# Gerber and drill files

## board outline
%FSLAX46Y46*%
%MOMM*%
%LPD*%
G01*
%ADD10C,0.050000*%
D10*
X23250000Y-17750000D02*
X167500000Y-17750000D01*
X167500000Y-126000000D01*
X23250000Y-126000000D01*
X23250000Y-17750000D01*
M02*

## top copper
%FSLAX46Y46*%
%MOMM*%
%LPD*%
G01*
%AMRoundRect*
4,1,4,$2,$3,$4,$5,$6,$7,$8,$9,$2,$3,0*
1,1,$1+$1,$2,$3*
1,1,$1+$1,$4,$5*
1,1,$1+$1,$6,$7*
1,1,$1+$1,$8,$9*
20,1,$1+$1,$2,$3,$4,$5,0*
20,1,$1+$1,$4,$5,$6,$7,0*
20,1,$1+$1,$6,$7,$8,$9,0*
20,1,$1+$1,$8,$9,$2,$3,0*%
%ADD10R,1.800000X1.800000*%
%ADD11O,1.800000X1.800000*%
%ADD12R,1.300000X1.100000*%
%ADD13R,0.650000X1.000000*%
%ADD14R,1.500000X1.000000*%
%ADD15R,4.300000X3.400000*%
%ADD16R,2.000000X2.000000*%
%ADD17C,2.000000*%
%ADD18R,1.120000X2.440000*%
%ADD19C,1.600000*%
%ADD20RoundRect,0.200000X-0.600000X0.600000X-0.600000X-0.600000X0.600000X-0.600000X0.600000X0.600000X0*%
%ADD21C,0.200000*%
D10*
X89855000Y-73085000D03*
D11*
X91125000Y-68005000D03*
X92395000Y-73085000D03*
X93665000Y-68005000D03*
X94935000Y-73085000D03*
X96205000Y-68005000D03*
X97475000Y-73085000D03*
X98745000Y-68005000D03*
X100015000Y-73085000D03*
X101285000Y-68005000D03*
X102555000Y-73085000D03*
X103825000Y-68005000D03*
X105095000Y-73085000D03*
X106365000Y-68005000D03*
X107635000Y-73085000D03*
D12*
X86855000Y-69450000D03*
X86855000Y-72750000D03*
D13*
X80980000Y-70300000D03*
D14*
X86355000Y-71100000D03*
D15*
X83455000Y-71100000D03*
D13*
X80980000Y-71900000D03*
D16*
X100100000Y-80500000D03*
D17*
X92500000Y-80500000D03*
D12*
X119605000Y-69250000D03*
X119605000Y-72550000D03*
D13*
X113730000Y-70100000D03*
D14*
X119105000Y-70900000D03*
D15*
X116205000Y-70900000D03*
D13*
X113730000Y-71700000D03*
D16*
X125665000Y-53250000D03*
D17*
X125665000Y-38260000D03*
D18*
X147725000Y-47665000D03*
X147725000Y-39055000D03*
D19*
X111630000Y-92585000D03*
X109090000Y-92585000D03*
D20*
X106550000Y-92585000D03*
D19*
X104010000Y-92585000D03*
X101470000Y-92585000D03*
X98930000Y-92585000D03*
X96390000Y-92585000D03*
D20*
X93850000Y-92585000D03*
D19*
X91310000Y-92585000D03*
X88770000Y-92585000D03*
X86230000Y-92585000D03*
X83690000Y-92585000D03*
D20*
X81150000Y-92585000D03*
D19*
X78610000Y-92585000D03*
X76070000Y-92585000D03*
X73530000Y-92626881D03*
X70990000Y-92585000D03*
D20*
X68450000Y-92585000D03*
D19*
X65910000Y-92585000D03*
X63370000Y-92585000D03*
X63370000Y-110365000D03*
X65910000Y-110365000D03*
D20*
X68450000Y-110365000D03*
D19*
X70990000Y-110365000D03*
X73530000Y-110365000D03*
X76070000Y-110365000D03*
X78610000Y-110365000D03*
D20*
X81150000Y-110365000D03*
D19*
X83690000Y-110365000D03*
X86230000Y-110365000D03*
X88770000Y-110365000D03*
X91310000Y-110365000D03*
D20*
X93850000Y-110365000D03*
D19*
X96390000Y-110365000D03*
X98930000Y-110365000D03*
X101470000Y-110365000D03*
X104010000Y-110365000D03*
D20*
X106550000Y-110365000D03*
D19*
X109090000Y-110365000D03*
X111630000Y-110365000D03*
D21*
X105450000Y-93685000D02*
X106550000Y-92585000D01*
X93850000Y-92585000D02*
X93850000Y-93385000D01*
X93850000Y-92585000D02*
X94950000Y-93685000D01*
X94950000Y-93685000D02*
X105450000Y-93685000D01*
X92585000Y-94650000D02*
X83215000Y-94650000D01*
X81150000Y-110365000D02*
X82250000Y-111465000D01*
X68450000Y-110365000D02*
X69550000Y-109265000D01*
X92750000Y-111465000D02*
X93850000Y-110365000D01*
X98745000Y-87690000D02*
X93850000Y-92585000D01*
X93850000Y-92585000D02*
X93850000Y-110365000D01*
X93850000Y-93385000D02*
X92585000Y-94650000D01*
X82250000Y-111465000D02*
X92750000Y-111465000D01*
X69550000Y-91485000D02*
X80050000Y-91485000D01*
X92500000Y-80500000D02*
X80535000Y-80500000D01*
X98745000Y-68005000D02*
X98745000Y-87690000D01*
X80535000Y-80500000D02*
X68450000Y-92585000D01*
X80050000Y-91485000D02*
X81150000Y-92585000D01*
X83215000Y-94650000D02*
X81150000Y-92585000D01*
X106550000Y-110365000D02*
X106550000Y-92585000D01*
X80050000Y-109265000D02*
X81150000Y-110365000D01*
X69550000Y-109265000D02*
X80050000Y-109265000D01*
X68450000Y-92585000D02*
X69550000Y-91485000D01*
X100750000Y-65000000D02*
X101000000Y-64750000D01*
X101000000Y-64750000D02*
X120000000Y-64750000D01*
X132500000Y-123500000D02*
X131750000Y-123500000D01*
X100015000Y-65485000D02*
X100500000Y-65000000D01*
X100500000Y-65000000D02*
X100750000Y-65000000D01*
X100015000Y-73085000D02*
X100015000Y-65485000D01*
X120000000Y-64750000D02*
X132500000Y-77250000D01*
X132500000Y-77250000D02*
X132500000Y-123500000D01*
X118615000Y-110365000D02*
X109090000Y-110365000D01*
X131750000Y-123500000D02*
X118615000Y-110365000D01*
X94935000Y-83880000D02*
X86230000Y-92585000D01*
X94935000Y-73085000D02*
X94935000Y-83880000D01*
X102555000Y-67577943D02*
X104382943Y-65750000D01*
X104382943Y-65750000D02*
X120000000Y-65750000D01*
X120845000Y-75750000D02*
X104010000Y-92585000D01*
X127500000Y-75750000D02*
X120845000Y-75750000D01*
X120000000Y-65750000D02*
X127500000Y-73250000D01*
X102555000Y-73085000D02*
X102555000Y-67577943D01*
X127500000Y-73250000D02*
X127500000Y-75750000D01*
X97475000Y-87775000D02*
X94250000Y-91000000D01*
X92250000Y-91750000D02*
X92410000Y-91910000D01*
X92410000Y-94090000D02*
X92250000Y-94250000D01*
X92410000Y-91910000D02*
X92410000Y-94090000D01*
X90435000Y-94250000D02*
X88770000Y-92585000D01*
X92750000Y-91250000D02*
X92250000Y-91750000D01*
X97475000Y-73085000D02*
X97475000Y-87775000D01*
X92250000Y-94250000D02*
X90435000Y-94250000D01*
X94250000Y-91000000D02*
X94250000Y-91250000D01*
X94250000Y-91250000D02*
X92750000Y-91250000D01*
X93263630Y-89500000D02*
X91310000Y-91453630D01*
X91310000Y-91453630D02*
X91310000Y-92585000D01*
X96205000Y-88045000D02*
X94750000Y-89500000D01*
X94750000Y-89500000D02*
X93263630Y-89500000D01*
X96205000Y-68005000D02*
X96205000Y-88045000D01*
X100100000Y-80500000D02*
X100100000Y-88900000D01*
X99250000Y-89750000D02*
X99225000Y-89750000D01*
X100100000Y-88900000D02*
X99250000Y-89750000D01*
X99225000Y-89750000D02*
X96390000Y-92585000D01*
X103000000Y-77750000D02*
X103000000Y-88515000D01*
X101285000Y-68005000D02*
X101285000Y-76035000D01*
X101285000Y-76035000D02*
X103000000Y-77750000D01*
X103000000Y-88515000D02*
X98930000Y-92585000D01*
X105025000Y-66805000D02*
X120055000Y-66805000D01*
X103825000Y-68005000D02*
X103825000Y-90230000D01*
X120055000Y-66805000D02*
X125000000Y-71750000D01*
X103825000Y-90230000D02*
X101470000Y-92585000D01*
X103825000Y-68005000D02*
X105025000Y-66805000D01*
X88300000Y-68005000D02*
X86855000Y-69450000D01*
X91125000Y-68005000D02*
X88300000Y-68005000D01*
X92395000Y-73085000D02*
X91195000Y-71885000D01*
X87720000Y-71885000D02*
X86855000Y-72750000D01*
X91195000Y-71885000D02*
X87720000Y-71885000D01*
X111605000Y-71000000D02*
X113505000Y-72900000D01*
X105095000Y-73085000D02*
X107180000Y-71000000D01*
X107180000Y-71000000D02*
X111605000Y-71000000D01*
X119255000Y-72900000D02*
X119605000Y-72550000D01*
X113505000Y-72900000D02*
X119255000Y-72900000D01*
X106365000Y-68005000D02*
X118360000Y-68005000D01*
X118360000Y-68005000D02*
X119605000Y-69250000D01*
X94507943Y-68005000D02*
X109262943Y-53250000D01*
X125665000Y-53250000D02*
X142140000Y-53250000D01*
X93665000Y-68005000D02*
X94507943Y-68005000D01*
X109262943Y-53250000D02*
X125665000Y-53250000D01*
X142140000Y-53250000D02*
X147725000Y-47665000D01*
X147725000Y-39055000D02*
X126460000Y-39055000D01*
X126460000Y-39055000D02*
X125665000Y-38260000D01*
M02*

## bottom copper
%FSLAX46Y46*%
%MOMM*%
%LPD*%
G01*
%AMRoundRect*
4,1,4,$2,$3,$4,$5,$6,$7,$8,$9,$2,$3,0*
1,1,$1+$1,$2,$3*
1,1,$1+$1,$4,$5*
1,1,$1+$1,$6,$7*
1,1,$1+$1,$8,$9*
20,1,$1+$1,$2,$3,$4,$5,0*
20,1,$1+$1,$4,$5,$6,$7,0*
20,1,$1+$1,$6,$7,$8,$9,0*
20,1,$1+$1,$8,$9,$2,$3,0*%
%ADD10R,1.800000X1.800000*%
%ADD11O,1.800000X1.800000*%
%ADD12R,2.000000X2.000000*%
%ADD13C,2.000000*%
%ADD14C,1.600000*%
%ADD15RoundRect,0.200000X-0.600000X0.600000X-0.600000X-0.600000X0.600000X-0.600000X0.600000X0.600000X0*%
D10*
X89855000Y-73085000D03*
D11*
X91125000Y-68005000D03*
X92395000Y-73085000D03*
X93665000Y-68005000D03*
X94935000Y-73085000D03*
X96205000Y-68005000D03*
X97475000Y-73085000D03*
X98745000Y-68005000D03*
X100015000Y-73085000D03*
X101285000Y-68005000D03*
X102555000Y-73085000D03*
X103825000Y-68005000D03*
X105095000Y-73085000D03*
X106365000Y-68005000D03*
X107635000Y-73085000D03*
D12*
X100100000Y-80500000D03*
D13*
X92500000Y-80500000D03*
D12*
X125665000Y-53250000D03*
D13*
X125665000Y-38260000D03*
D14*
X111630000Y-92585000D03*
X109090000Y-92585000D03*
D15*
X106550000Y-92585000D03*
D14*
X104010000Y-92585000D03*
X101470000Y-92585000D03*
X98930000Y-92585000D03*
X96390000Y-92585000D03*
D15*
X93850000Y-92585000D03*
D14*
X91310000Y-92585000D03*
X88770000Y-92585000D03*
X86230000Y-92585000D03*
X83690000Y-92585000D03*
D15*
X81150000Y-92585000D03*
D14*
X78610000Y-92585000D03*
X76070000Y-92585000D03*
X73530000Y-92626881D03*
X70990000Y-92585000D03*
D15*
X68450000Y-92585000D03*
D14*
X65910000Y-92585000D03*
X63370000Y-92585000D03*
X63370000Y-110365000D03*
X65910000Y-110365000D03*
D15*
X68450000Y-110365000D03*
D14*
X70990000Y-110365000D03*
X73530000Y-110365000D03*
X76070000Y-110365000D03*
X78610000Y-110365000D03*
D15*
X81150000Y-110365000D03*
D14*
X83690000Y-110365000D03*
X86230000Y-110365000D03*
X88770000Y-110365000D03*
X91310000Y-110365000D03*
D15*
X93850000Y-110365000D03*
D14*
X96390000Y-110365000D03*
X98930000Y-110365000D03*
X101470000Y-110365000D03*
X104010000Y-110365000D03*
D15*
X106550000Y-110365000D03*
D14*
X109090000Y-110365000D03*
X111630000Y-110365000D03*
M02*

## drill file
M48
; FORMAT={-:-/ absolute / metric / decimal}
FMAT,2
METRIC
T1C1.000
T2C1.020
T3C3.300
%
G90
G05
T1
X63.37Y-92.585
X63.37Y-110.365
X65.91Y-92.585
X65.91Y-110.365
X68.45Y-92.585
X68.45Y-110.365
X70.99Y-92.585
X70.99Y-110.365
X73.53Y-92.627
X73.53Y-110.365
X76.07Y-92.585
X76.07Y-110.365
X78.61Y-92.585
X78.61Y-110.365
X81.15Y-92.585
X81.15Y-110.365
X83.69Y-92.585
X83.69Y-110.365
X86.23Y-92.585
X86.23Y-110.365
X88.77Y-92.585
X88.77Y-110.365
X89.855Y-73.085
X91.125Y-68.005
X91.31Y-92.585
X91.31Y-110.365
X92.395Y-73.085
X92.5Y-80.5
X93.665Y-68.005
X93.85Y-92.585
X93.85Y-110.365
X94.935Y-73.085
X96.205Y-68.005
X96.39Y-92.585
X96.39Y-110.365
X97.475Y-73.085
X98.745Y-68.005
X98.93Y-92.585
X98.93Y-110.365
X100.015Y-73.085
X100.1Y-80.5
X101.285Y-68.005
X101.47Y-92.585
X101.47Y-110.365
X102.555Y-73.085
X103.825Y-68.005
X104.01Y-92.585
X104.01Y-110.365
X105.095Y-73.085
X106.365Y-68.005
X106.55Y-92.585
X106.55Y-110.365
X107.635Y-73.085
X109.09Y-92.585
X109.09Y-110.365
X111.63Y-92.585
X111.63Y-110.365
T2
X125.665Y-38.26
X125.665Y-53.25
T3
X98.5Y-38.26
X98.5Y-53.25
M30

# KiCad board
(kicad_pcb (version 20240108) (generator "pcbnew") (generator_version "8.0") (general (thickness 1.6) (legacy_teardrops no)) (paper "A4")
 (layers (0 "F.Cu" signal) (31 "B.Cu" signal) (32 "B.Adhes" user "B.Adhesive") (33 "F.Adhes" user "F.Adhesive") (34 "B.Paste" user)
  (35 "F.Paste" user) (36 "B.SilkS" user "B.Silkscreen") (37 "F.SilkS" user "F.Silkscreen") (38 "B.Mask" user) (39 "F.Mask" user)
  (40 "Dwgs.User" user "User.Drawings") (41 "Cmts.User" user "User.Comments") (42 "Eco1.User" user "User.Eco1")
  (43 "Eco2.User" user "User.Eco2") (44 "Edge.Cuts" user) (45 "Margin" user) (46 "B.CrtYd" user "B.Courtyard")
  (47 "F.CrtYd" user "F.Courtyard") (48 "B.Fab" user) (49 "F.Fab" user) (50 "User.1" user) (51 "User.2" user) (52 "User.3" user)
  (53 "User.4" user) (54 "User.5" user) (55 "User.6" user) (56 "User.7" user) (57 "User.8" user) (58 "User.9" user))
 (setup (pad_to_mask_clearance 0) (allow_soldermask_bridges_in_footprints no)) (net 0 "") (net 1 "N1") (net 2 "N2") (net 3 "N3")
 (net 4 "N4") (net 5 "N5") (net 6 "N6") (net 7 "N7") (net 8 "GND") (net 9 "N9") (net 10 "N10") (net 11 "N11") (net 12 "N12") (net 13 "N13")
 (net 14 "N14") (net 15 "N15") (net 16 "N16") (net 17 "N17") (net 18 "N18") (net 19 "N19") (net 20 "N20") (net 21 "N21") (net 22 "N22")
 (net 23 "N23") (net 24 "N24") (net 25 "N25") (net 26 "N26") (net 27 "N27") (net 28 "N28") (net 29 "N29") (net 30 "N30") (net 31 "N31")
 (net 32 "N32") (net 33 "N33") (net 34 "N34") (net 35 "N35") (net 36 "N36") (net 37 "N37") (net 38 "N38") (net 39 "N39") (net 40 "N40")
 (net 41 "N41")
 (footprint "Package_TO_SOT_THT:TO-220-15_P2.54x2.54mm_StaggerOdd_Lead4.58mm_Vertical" (layer "F.Cu") (at 89.855 73.085)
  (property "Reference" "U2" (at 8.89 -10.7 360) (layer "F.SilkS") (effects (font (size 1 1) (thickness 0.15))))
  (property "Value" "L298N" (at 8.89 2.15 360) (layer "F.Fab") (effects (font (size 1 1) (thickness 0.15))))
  (pad "1" thru_hole rect (at 0 0) (size 1.8 1.8) (drill 1) (layers "*.Cu" "*.Mask") (remove_unused_layers no) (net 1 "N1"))
  (pad "2" thru_hole oval (at 1.27 -5.08) (size 1.8 1.8) (drill 1) (layers "*.Cu" "*.Mask") (remove_unused_layers no) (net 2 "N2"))
  (pad "3" thru_hole oval (at 2.54 0) (size 1.8 1.8) (drill 1) (layers "*.Cu" "*.Mask") (remove_unused_layers no) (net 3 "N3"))
  (pad "4" thru_hole oval (at 3.81 -5.08) (size 1.8 1.8) (drill 1) (layers "*.Cu" "*.Mask") (remove_unused_layers no) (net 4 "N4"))
  (pad "5" thru_hole oval (at 5.08 0) (size 1.8 1.8) (drill 1) (layers "*.Cu" "*.Mask") (remove_unused_layers no) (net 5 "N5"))
  (pad "6" thru_hole oval (at 6.35 -5.08) (size 1.8 1.8) (drill 1) (layers "*.Cu" "*.Mask") (remove_unused_layers no) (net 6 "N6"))
  (pad "7" thru_hole oval (at 7.62 0) (size 1.8 1.8) (drill 1) (layers "*.Cu" "*.Mask") (remove_unused_layers no) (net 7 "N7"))
  (pad "8" thru_hole oval (at 8.89 -5.08) (size 1.8 1.8) (drill 1) (layers "*.Cu" "*.Mask") (remove_unused_layers no) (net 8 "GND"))
  (pad "9" thru_hole oval (at 10.16 0) (size 1.8 1.8) (drill 1) (layers "*.Cu" "*.Mask") (remove_unused_layers no) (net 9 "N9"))
  (pad "10" thru_hole oval (at 11.43 -5.08) (size 1.8 1.8) (drill 1) (layers "*.Cu" "*.Mask") (remove_unused_layers no) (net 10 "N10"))
  (pad "11" thru_hole oval (at 12.7 0) (size 1.8 1.8) (drill 1) (layers "*.Cu" "*.Mask") (remove_unused_layers no) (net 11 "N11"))
  (pad "12" thru_hole oval (at 13.97 -5.08) (size 1.8 1.8) (drill 1) (layers "*.Cu" "*.Mask") (remove_unused_layers no) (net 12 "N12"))
  (pad "13" thru_hole oval (at 15.24 0) (size 1.8 1.8) (drill 1) (layers "*.Cu" "*.Mask") (remove_unused_layers no) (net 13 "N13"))
  (pad "14" thru_hole oval (at 16.51 -5.08) (size 1.8 1.8) (drill 1) (layers "*.Cu" "*.Mask") (remove_unused_layers no) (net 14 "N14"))
  (pad "15" thru_hole oval (at 17.78 0) (size 1.8 1.8) (drill 1) (layers "*.Cu" "*.Mask") (remove_unused_layers no) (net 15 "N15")))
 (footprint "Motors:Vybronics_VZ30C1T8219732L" (layer "F.Cu") (at 82.505 71.1 -90)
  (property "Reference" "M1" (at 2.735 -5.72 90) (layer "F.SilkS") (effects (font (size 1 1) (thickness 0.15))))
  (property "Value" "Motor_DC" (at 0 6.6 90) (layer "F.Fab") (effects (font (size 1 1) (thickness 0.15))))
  (pad "" smd rect (at -0.85 -2.315 180) (size 1.07 1.4) (layers "F.Paste"))
  (pad "" smd rect (at -0.85 -0.905 180) (size 1.07 1.4) (layers "F.Paste"))
  (pad "" smd rect (at -0.85 0.505 180) (size 1.07 1.4) (layers "F.Paste"))
  (pad "" smd rect (at 0.85 -2.315 180) (size 1.07 1.4) (layers "F.Paste"))
  (pad "" smd rect (at 0.85 -0.905 180) (size 1.07 1.4) (layers "F.Paste"))
  (pad "" smd rect (at 0.85 0.505 180) (size 1.07 1.4) (layers "F.Paste"))
  (pad "1" smd rect (at -1.65 -4.35 180) (size 1.3 1.1) (layers "F.Cu" "F.Paste" "F.Mask") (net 2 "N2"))
  (pad "2" smd rect (at 1.65 -4.35 180) (size 1.3 1.1) (layers "F.Cu" "F.Paste" "F.Mask") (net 3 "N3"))
  (pad "SH" smd rect (at -0.8 1.525 270) (size 1 0.65) (layers "F.Cu" "F.Paste" "F.Mask"))
  (pad "SH" smd rect (at 0 -3.85 180) (size 1.5 1) (layers "F.Cu" "F.Paste" "F.Mask"))
  (pad "SH" smd rect (at 0 -0.95 180) (size 4.3 3.4) (layers "F.Cu" "F.Mask"))
  (pad "SH" smd rect (at 0.8 1.525 270) (size 1 0.65) (layers "F.Cu" "F.Paste" "F.Mask")))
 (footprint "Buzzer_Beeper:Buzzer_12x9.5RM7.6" (layer "F.Cu") (at 100.1 80.5 180)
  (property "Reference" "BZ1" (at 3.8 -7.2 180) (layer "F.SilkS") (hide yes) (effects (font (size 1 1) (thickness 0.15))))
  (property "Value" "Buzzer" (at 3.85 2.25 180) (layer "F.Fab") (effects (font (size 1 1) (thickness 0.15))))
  (pad "1" thru_hole rect (at 0 0 180) (size 2 2) (drill 1) (layers "*.Cu" "*.Mask") (remove_unused_layers no) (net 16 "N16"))
  (pad "2" thru_hole circle (at 7.6 0 180) (size 2 2) (drill 1) (layers "*.Cu" "*.Mask") (remove_unused_layers no) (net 8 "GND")))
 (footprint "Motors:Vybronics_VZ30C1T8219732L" (layer "F.Cu") (at 115.255 70.9 -90)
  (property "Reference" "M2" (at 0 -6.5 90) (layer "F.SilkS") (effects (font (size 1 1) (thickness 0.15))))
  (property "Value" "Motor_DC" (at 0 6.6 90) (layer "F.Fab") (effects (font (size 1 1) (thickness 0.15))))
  (pad "" smd rect (at -0.85 -2.315 180) (size 1.07 1.4) (layers "F.Paste"))
  (pad "" smd rect (at -0.85 -0.905 180) (size 1.07 1.4) (layers "F.Paste"))
  (pad "" smd rect (at -0.85 0.505 180) (size 1.07 1.4) (layers "F.Paste"))
  (pad "" smd rect (at 0.85 -2.315 180) (size 1.07 1.4) (layers "F.Paste"))
  (pad "" smd rect (at 0.85 -0.905 180) (size 1.07 1.4) (layers "F.Paste"))
  (pad "" smd rect (at 0.85 0.505 180) (size 1.07 1.4) (layers "F.Paste"))
  (pad "1" smd rect (at -1.65 -4.35 180) (size 1.3 1.1) (layers "F.Cu" "F.Paste" "F.Mask") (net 14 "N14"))
  (pad "2" smd rect (at 1.65 -4.35 180) (size 1.3 1.1) (layers "F.Cu" "F.Paste" "F.Mask") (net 13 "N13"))
  (pad "SH" smd rect (at -0.8 1.525 270) (size 1 0.65) (layers "F.Cu" "F.Paste" "F.Mask"))
  (pad "SH" smd rect (at 0 -3.85 180) (size 1.5 1) (layers "F.Cu" "F.Paste" "F.Mask"))
  (pad "SH" smd rect (at 0 -0.95 180) (size 4.3 3.4) (layers "F.Cu" "F.Mask"))
  (pad "SH" smd rect (at 0.8 1.525 270) (size 1 0.65) (layers "F.Cu" "F.Paste" "F.Mask")))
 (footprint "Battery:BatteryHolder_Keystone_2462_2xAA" (layer "F.Cu") (at 125.665 53.25 180)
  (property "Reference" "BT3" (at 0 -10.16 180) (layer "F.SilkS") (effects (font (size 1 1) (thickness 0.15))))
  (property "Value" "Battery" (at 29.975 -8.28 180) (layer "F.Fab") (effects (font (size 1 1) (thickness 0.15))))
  (pad "" np_thru_hole circle (at 27.165 0 180) (size 3.3 3.3) (drill 3.3) (layers "*.Cu" "*.Mask"))
  (pad "" np_thru_hole circle (at 27.165 14.99 180) (size 3.3 3.3) (drill 3.3) (layers "*.Cu" "*.Mask"))
  (pad "1" thru_hole rect (at 0 0 180) (size 2 2) (drill 1.02) (layers "*.Cu" "*.Mask") (remove_unused_layers no) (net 4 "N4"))
  (pad "2" thru_hole circle (at 0 14.99 180) (size 2 2) (drill 1.02) (layers "*.Cu" "*.Mask") (remove_unused_layers no) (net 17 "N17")))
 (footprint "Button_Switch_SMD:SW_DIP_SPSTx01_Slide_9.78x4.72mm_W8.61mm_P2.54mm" (layer "F.Cu") (at 147.725 43.36 90)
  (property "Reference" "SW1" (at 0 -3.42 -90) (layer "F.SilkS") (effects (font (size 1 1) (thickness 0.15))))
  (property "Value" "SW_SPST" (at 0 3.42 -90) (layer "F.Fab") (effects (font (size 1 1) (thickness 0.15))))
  (pad "1" smd rect (at -4.305 0 90) (size 2.44 1.12) (layers "F.Cu" "F.Paste" "F.Mask") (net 4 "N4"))
  (pad "2" smd rect (at 4.305 0 90) (size 2.44 1.12) (layers "F.Cu" "F.Paste" "F.Mask") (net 17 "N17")))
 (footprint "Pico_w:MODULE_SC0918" (layer "F.Cu") (at 87.5 101.475 -90)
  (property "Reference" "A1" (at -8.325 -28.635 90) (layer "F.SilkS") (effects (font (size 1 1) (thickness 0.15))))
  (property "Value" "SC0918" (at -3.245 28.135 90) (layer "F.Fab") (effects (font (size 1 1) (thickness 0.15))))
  (pad "1" thru_hole circle (at -8.89 -24.13 270) (size 1.6 1.6) (drill 1) (layers "*.Cu" "*.Mask") (remove_unused_layers no) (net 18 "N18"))
  (pad "2" thru_hole circle (at -8.89 -21.59 270) (size 1.6 1.6) (drill 1) (layers "*.Cu" "*.Mask") (remove_unused_layers no) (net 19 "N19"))
  (pad "3" thru_hole roundrect (at -8.89 -19.05 270) (size 1.6 1.6) (drill 1) (layers "*.Cu" "*.Mask") (remove_unused_layers no)
   (roundrect_rratio 0.125) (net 8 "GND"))
  (pad "4" thru_hole circle (at -8.89 -16.51 270) (size 1.6 1.6) (drill 1) (layers "*.Cu" "*.Mask") (remove_unused_layers no) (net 11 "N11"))
  (pad "5" thru_hole circle (at -8.89 -13.97 270) (size 1.6 1.6) (drill 1) (layers "*.Cu" "*.Mask") (remove_unused_layers no) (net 12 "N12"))
  (pad "6" thru_hole circle (at -8.89 -11.43 270) (size 1.6 1.6) (drill 1) (layers "*.Cu" "*.Mask") (remove_unused_layers no) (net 10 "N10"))
  (pad "7" thru_hole circle (at -8.89 -8.89 270) (size 1.6 1.6) (drill 1) (layers "*.Cu" "*.Mask") (remove_unused_layers no) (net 16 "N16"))
  (pad "8" thru_hole roundrect (at -8.89 -6.35 270) (size 1.6 1.6) (drill 1) (layers "*.Cu" "*.Mask") (remove_unused_layers no)
   (roundrect_rratio 0.125) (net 8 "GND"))
  (pad "9" thru_hole circle (at -8.89 -3.81 270) (size 1.6 1.6) (drill 1) (layers "*.Cu" "*.Mask") (remove_unused_layers no) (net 6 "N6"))
  (pad "10" thru_hole circle (at -8.89 -1.27 270) (size 1.6 1.6) (drill 1) (layers "*.Cu" "*.Mask") (remove_unused_layers no) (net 7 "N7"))
  (pad "11" thru_hole circle (at -8.89 1.27 270) (size 1.6 1.6) (drill 1) (layers "*.Cu" "*.Mask") (remove_unused_layers no) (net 5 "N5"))
  (pad "12" thru_hole circle (at -8.89 3.81 270) (size 1.6 1.6) (drill 1) (layers "*.Cu" "*.Mask") (remove_unused_layers no) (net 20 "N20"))
  (pad "13" thru_hole roundrect (at -8.89 6.35 270) (size 1.6 1.6) (drill 1) (layers "*.Cu" "*.Mask") (remove_unused_layers no)
   (roundrect_rratio 0.125) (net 8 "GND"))
  (pad "14" thru_hole circle (at -8.89 8.89 270) (size 1.6 1.6) (drill 1) (layers "*.Cu" "*.Mask") (remove_unused_layers no) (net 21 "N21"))
  (pad "15" thru_hole circle (at -8.89 11.43 270) (size 1.6 1.6) (drill 1) (layers "*.Cu" "*.Mask") (remove_unused_layers no) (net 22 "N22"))
  (pad "16" thru_hole circle (at -8.848119 13.97 270) (size 1.6 1.6) (drill 1) (layers "*.Cu" "*.Mask") (remove_unused_layers no)
   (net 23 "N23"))
  (pad "17" thru_hole circle (at -8.89 16.51 270) (size 1.6 1.6) (drill 1) (layers "*.Cu" "*.Mask") (remove_unused_layers no) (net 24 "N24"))
  (pad "18" thru_hole roundrect (at -8.89 19.05 270) (size 1.6 1.6) (drill 1) (layers "*.Cu" "*.Mask") (remove_unused_layers no)
   (roundrect_rratio 0.125) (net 8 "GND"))
  (pad "19" thru_hole circle (at -8.89 21.59 270) (size 1.6 1.6) (drill 1) (layers "*.Cu" "*.Mask") (remove_unused_layers no) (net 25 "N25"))
  (pad "20" thru_hole circle (at -8.89 24.13 270) (size 1.6 1.6) (drill 1) (layers "*.Cu" "*.Mask") (remove_unused_layers no) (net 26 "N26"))
  (pad "21" thru_hole circle (at 8.89 24.13 270) (size 1.6 1.6) (drill 1) (layers "*.Cu" "*.Mask") (remove_unused_layers no) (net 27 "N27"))
  (pad "22" thru_hole circle (at 8.89 21.59 270) (size 1.6 1.6) (drill 1) (layers "*.Cu" "*.Mask") (remove_unused_layers no) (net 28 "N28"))
  (pad "23" thru_hole roundrect (at 8.89 19.05 270) (size 1.6 1.6) (drill 1) (layers "*.Cu" "*.Mask") (remove_unused_layers no)
   (roundrect_rratio 0.125) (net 8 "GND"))
  (pad "24" thru_hole circle (at 8.89 16.51 270) (size 1.6 1.6) (drill 1) (layers "*.Cu" "*.Mask") (remove_unused_layers no) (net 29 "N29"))
  (pad "25" thru_hole circle (at 8.89 13.97 270) (size 1.6 1.6) (drill 1) (layers "*.Cu" "*.Mask") (remove_unused_layers no) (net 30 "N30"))
  (pad "26" thru_hole circle (at 8.89 11.43 270) (size 1.6 1.6) (drill 1) (layers "*.Cu" "*.Mask") (remove_unused_layers no) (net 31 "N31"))
  (pad "27" thru_hole circle (at 8.89 8.89 270) (size 1.6 1.6) (drill 1) (layers "*.Cu" "*.Mask") (remove_unused_layers no) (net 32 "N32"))
  (pad "28" thru_hole roundrect (at 8.89 6.35 270) (size 1.6 1.6) (drill 1) (layers "*.Cu" "*.Mask") (remove_unused_layers no)
   (roundrect_rratio 0.125) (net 8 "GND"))
  (pad "29" thru_hole circle (at 8.89 3.81 270) (size 1.6 1.6) (drill 1) (layers "*.Cu" "*.Mask") (remove_unused_layers no) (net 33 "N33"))
  (pad "30" thru_hole circle (at 8.89 1.27 270) (size 1.6 1.6) (drill 1) (layers "*.Cu" "*.Mask") (remove_unused_layers no) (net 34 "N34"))
  (pad "31" thru_hole circle (at 8.89 -1.27 270) (size 1.6 1.6) (drill 1) (layers "*.Cu" "*.Mask") (remove_unused_layers no) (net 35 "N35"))
  (pad "32" thru_hole circle (at 8.89 -3.81 270) (size 1.6 1.6) (drill 1) (layers "*.Cu" "*.Mask") (remove_unused_layers no) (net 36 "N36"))
  (pad "33" thru_hole roundrect (at 8.89 -6.35 270) (size 1.6 1.6) (drill 1) (layers "*.Cu" "*.Mask") (remove_unused_layers no)
   (roundrect_rratio 0.125) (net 8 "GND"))
  (pad "34" thru_hole circle (at 8.89 -8.89 270) (size 1.6 1.6) (drill 1) (layers "*.Cu" "*.Mask") (remove_unused_layers no) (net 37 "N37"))
  (pad "35" thru_hole circle (at 8.89 -11.43 270) (size 1.6 1.6) (drill 1) (layers "*.Cu" "*.Mask") (remove_unused_layers no) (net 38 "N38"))
  (pad "36" thru_hole circle (at 8.89 -13.97 270) (size 1.6 1.6) (drill 1) (layers "*.Cu" "*.Mask") (remove_unused_layers no) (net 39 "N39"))
  (pad "37" thru_hole circle (at 8.89 -16.51 270) (size 1.6 1.6) (drill 1) (layers "*.Cu" "*.Mask") (remove_unused_layers no) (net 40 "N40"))
  (pad "38" thru_hole roundrect (at 8.89 -19.05 270) (size 1.6 1.6) (drill 1) (layers "*.Cu" "*.Mask") (remove_unused_layers no)
   (roundrect_rratio 0.125) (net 8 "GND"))
  (pad "39" thru_hole circle (at 8.89 -21.59 270) (size 1.6 1.6) (drill 1) (layers "*.Cu" "*.Mask") (remove_unused_layers no) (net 9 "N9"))
  (pad "40" thru_hole circle (at 8.89 -24.13 270) (size 1.6 1.6) (drill 1) (layers "*.Cu" "*.Mask") (remove_unused_layers no) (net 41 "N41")))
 (gr_rect (start 23.25 17.75) (end 167.5 126) (stroke (width 0.05) (type default)) (fill none) (layer "Edge.Cuts"))
 (segment (start 105.45 93.685) (end 106.55 92.585) (width 0.2) (layer "F.Cu") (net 8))
 (segment (start 93.85 92.585) (end 93.85 93.385) (width 0.2) (layer "F.Cu") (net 8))
 (segment (start 93.85 92.585) (end 94.95 93.685) (width 0.2) (layer "F.Cu") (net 8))
 (segment (start 94.95 93.685) (end 105.45 93.685) (width 0.2) (layer "F.Cu") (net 8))
 (segment (start 92.585 94.65) (end 83.215 94.65) (width 0.2) (layer "F.Cu") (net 8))
 (segment (start 81.15 110.365) (end 82.25 111.465) (width 0.2) (layer "F.Cu") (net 8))
 (segment (start 68.45 110.365) (end 69.55 109.265) (width 0.2) (layer "F.Cu") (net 8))
 (segment (start 92.75 111.465) (end 93.85 110.365) (width 0.2) (layer "F.Cu") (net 8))
 (segment (start 98.745 87.69) (end 93.85 92.585) (width 0.2) (layer "F.Cu") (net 8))
 (segment (start 93.85 92.585) (end 93.85 110.365) (width 0.2) (layer "F.Cu") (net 8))
 (segment (start 93.85 93.385) (end 92.585 94.65) (width 0.2) (layer "F.Cu") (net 8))
 (segment (start 82.25 111.465) (end 92.75 111.465) (width 0.2) (layer "F.Cu") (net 8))
 (segment (start 69.55 91.485) (end 80.05 91.485) (width 0.2) (layer "F.Cu") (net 8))
 (segment (start 92.5 80.5) (end 80.535 80.5) (width 0.2) (layer "F.Cu") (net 8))
 (segment (start 98.745 68.005) (end 98.745 87.69) (width 0.2) (layer "F.Cu") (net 8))
 (segment (start 80.535 80.5) (end 68.45 92.585) (width 0.2) (layer "F.Cu") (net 8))
 (segment (start 80.05 91.485) (end 81.15 92.585) (width 0.2) (layer "F.Cu") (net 8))
 (segment (start 83.215 94.65) (end 81.15 92.585) (width 0.2) (layer "F.Cu") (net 8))
 (segment (start 106.55 110.365) (end 106.55 92.585) (width 0.2) (layer "F.Cu") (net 8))
 (segment (start 80.05 109.265) (end 81.15 110.365) (width 0.2) (layer "F.Cu") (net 8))
 (segment (start 69.55 109.265) (end 80.05 109.265) (width 0.2) (layer "F.Cu") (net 8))
 (segment (start 68.45 92.585) (end 69.55 91.485) (width 0.2) (layer "F.Cu") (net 8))
 (segment (start 100.75 65) (end 101 64.75) (width 0.2) (layer "F.Cu") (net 9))
 (segment (start 101 64.75) (end 120 64.75) (width 0.2) (layer "F.Cu") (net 9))
 (segment (start 132.5 123.5) (end 131.75 123.5) (width 0.2) (layer "F.Cu") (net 9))
 (segment (start 100.015 65.485) (end 100.5 65) (width 0.2) (layer "F.Cu") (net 9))
 (segment (start 100.5 65) (end 100.75 65) (width 0.2) (layer "F.Cu") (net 9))
 (segment (start 100.015 73.085) (end 100.015 65.485) (width 0.2) (layer "F.Cu") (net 9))
 (segment (start 120 64.75) (end 132.5 77.25) (width 0.2) (layer "F.Cu") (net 9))
 (segment (start 132.5 77.25) (end 132.5 123.5) (width 0.2) (layer "F.Cu") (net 9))
 (segment (start 118.615 110.365) (end 109.09 110.365) (width 0.2) (layer "F.Cu") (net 9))
 (segment (start 131.75 123.5) (end 118.615 110.365) (width 0.2) (layer "F.Cu") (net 9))
 (segment (start 94.935 83.88) (end 86.23 92.585) (width 0.2) (layer "F.Cu") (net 5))
 (segment (start 94.935 73.085) (end 94.935 83.88) (width 0.2) (layer "F.Cu") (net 5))
 (segment (start 102.555 67.577943) (end 104.382943 65.75) (width 0.2) (layer "F.Cu") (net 11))
 (segment (start 104.382943 65.75) (end 120 65.75) (width 0.2) (layer "F.Cu") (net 11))
 (segment (start 120.845 75.75) (end 104.01 92.585) (width 0.2) (layer "F.Cu") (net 11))
 (segment (start 127.5 75.75) (end 120.845 75.75) (width 0.2) (layer "F.Cu") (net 11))
 (segment (start 120 65.75) (end 127.5 73.25) (width 0.2) (layer "F.Cu") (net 11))
 (segment (start 102.555 73.085) (end 102.555 67.577943) (width 0.2) (layer "F.Cu") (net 11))
 (segment (start 127.5 73.25) (end 127.5 75.75) (width 0.2) (layer "F.Cu") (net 11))
 (segment (start 97.475 87.775) (end 94.25 91) (width 0.2) (layer "F.Cu") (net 7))
 (segment (start 92.25 91.75) (end 92.41 91.91) (width 0.2) (layer "F.Cu") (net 7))
 (segment (start 92.41 94.09) (end 92.25 94.25) (width 0.2) (layer "F.Cu") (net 7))
 (segment (start 92.41 91.91) (end 92.41 94.09) (width 0.2) (layer "F.Cu") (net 7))
 (segment (start 90.435 94.25) (end 88.77 92.585) (width 0.2) (layer "F.Cu") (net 7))
 (segment (start 92.75 91.25) (end 92.25 91.75) (width 0.2) (layer "F.Cu") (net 7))
 (segment (start 97.475 73.085) (end 97.475 87.775) (width 0.2) (layer "F.Cu") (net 7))
 (segment (start 92.25 94.25) (end 90.435 94.25) (width 0.2) (layer "F.Cu") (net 7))
 (segment (start 94.25 91) (end 94.25 91.25) (width 0.2) (layer "F.Cu") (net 7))
 (segment (start 94.25 91.25) (end 92.75 91.25) (width 0.2) (layer "F.Cu") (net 7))
 (segment (start 93.26363 89.5) (end 91.31 91.45363) (width 0.2) (layer "F.Cu") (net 6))
 (segment (start 91.31 91.45363) (end 91.31 92.585) (width 0.2) (layer "F.Cu") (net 6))
 (segment (start 96.205 88.045) (end 94.75 89.5) (width 0.2) (layer "F.Cu") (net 6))
 (segment (start 94.75 89.5) (end 93.26363 89.5) (width 0.2) (layer "F.Cu") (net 6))
 (segment (start 96.205 68.005) (end 96.205 88.045) (width 0.2) (layer "F.Cu") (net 6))
 (segment (start 100.1 80.5) (end 100.1 88.9) (width 0.2) (layer "F.Cu") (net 16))
 (segment (start 99.25 89.75) (end 99.225 89.75) (width 0.2) (layer "F.Cu") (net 16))
 (segment (start 100.1 88.9) (end 99.25 89.75) (width 0.2) (layer "F.Cu") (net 16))
 (segment (start 99.225 89.75) (end 96.39 92.585) (width 0.2) (layer "F.Cu") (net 16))
 (segment (start 103 77.75) (end 103 88.515) (width 0.2) (layer "F.Cu") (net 10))
 (segment (start 101.285 68.005) (end 101.285 76.035) (width 0.2) (layer "F.Cu") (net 10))
 (segment (start 101.285 76.035) (end 103 77.75) (width 0.2) (layer "F.Cu") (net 10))
 (segment (start 103 88.515) (end 98.93 92.585) (width 0.2) (layer "F.Cu") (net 10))
 (segment (start 105.025 66.805) (end 120.055 66.805) (width 0.2) (layer "F.Cu") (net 12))
 (segment (start 103.825 68.005) (end 103.825 90.23) (width 0.2) (layer "F.Cu") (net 12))
 (segment (start 120.055 66.805) (end 125 71.75) (width 0.2) (layer "F.Cu") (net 12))
 (segment (start 103.825 90.23) (end 101.47 92.585) (width 0.2) (layer "F.Cu") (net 12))
 (segment (start 103.825 68.005) (end 105.025 66.805) (width 0.2) (layer "F.Cu") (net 12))
 (segment (start 88.3 68.005) (end 86.855 69.45) (width 0.2) (layer "F.Cu") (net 2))
 (segment (start 91.125 68.005) (end 88.3 68.005) (width 0.2) (layer "F.Cu") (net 2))
 (segment (start 92.395 73.085) (end 91.195 71.885) (width 0.2) (layer "F.Cu") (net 3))
 (segment (start 87.72 71.885) (end 86.855 72.75) (width 0.2) (layer "F.Cu") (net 3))
 (segment (start 91.195 71.885) (end 87.72 71.885) (width 0.2) (layer "F.Cu") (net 3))
 (segment (start 111.605 71) (end 113.505 72.9) (width 0.2) (layer "F.Cu") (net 13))
 (segment (start 105.095 73.085) (end 107.18 71) (width 0.2) (layer "F.Cu") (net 13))
 (segment (start 107.18 71) (end 111.605 71) (width 0.2) (layer "F.Cu") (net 13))
 (segment (start 119.255 72.9) (end 119.605 72.55) (width 0.2) (layer "F.Cu") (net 13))
 (segment (start 113.505 72.9) (end 119.255 72.9) (width 0.2) (layer "F.Cu") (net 13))
 (segment (start 106.365 68.005) (end 118.36 68.005) (width 0.2) (layer "F.Cu") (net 14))
 (segment (start 118.36 68.005) (end 119.605 69.25) (width 0.2) (layer "F.Cu") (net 14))
 (segment (start 94.507943 68.005) (end 109.262943 53.25) (width 0.2) (layer "F.Cu") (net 4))
 (segment (start 125.665 53.25) (end 142.14 53.25) (width 0.2) (layer "F.Cu") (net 4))
 (segment (start 93.665 68.005) (end 94.507943 68.005) (width 0.2) (layer "F.Cu") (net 4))
 (segment (start 109.262943 53.25) (end 125.665 53.25) (width 0.2) (layer "F.Cu") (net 4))
 (segment (start 142.14 53.25) (end 147.725 47.665) (width 0.2) (layer "F.Cu") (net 4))
 (segment (start 147.725 39.055) (end 126.46 39.055) (width 0.2) (layer "F.Cu") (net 17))
 (segment (start 126.46 39.055) (end 125.665 38.26) (width 0.2) (layer "F.Cu") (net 17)))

